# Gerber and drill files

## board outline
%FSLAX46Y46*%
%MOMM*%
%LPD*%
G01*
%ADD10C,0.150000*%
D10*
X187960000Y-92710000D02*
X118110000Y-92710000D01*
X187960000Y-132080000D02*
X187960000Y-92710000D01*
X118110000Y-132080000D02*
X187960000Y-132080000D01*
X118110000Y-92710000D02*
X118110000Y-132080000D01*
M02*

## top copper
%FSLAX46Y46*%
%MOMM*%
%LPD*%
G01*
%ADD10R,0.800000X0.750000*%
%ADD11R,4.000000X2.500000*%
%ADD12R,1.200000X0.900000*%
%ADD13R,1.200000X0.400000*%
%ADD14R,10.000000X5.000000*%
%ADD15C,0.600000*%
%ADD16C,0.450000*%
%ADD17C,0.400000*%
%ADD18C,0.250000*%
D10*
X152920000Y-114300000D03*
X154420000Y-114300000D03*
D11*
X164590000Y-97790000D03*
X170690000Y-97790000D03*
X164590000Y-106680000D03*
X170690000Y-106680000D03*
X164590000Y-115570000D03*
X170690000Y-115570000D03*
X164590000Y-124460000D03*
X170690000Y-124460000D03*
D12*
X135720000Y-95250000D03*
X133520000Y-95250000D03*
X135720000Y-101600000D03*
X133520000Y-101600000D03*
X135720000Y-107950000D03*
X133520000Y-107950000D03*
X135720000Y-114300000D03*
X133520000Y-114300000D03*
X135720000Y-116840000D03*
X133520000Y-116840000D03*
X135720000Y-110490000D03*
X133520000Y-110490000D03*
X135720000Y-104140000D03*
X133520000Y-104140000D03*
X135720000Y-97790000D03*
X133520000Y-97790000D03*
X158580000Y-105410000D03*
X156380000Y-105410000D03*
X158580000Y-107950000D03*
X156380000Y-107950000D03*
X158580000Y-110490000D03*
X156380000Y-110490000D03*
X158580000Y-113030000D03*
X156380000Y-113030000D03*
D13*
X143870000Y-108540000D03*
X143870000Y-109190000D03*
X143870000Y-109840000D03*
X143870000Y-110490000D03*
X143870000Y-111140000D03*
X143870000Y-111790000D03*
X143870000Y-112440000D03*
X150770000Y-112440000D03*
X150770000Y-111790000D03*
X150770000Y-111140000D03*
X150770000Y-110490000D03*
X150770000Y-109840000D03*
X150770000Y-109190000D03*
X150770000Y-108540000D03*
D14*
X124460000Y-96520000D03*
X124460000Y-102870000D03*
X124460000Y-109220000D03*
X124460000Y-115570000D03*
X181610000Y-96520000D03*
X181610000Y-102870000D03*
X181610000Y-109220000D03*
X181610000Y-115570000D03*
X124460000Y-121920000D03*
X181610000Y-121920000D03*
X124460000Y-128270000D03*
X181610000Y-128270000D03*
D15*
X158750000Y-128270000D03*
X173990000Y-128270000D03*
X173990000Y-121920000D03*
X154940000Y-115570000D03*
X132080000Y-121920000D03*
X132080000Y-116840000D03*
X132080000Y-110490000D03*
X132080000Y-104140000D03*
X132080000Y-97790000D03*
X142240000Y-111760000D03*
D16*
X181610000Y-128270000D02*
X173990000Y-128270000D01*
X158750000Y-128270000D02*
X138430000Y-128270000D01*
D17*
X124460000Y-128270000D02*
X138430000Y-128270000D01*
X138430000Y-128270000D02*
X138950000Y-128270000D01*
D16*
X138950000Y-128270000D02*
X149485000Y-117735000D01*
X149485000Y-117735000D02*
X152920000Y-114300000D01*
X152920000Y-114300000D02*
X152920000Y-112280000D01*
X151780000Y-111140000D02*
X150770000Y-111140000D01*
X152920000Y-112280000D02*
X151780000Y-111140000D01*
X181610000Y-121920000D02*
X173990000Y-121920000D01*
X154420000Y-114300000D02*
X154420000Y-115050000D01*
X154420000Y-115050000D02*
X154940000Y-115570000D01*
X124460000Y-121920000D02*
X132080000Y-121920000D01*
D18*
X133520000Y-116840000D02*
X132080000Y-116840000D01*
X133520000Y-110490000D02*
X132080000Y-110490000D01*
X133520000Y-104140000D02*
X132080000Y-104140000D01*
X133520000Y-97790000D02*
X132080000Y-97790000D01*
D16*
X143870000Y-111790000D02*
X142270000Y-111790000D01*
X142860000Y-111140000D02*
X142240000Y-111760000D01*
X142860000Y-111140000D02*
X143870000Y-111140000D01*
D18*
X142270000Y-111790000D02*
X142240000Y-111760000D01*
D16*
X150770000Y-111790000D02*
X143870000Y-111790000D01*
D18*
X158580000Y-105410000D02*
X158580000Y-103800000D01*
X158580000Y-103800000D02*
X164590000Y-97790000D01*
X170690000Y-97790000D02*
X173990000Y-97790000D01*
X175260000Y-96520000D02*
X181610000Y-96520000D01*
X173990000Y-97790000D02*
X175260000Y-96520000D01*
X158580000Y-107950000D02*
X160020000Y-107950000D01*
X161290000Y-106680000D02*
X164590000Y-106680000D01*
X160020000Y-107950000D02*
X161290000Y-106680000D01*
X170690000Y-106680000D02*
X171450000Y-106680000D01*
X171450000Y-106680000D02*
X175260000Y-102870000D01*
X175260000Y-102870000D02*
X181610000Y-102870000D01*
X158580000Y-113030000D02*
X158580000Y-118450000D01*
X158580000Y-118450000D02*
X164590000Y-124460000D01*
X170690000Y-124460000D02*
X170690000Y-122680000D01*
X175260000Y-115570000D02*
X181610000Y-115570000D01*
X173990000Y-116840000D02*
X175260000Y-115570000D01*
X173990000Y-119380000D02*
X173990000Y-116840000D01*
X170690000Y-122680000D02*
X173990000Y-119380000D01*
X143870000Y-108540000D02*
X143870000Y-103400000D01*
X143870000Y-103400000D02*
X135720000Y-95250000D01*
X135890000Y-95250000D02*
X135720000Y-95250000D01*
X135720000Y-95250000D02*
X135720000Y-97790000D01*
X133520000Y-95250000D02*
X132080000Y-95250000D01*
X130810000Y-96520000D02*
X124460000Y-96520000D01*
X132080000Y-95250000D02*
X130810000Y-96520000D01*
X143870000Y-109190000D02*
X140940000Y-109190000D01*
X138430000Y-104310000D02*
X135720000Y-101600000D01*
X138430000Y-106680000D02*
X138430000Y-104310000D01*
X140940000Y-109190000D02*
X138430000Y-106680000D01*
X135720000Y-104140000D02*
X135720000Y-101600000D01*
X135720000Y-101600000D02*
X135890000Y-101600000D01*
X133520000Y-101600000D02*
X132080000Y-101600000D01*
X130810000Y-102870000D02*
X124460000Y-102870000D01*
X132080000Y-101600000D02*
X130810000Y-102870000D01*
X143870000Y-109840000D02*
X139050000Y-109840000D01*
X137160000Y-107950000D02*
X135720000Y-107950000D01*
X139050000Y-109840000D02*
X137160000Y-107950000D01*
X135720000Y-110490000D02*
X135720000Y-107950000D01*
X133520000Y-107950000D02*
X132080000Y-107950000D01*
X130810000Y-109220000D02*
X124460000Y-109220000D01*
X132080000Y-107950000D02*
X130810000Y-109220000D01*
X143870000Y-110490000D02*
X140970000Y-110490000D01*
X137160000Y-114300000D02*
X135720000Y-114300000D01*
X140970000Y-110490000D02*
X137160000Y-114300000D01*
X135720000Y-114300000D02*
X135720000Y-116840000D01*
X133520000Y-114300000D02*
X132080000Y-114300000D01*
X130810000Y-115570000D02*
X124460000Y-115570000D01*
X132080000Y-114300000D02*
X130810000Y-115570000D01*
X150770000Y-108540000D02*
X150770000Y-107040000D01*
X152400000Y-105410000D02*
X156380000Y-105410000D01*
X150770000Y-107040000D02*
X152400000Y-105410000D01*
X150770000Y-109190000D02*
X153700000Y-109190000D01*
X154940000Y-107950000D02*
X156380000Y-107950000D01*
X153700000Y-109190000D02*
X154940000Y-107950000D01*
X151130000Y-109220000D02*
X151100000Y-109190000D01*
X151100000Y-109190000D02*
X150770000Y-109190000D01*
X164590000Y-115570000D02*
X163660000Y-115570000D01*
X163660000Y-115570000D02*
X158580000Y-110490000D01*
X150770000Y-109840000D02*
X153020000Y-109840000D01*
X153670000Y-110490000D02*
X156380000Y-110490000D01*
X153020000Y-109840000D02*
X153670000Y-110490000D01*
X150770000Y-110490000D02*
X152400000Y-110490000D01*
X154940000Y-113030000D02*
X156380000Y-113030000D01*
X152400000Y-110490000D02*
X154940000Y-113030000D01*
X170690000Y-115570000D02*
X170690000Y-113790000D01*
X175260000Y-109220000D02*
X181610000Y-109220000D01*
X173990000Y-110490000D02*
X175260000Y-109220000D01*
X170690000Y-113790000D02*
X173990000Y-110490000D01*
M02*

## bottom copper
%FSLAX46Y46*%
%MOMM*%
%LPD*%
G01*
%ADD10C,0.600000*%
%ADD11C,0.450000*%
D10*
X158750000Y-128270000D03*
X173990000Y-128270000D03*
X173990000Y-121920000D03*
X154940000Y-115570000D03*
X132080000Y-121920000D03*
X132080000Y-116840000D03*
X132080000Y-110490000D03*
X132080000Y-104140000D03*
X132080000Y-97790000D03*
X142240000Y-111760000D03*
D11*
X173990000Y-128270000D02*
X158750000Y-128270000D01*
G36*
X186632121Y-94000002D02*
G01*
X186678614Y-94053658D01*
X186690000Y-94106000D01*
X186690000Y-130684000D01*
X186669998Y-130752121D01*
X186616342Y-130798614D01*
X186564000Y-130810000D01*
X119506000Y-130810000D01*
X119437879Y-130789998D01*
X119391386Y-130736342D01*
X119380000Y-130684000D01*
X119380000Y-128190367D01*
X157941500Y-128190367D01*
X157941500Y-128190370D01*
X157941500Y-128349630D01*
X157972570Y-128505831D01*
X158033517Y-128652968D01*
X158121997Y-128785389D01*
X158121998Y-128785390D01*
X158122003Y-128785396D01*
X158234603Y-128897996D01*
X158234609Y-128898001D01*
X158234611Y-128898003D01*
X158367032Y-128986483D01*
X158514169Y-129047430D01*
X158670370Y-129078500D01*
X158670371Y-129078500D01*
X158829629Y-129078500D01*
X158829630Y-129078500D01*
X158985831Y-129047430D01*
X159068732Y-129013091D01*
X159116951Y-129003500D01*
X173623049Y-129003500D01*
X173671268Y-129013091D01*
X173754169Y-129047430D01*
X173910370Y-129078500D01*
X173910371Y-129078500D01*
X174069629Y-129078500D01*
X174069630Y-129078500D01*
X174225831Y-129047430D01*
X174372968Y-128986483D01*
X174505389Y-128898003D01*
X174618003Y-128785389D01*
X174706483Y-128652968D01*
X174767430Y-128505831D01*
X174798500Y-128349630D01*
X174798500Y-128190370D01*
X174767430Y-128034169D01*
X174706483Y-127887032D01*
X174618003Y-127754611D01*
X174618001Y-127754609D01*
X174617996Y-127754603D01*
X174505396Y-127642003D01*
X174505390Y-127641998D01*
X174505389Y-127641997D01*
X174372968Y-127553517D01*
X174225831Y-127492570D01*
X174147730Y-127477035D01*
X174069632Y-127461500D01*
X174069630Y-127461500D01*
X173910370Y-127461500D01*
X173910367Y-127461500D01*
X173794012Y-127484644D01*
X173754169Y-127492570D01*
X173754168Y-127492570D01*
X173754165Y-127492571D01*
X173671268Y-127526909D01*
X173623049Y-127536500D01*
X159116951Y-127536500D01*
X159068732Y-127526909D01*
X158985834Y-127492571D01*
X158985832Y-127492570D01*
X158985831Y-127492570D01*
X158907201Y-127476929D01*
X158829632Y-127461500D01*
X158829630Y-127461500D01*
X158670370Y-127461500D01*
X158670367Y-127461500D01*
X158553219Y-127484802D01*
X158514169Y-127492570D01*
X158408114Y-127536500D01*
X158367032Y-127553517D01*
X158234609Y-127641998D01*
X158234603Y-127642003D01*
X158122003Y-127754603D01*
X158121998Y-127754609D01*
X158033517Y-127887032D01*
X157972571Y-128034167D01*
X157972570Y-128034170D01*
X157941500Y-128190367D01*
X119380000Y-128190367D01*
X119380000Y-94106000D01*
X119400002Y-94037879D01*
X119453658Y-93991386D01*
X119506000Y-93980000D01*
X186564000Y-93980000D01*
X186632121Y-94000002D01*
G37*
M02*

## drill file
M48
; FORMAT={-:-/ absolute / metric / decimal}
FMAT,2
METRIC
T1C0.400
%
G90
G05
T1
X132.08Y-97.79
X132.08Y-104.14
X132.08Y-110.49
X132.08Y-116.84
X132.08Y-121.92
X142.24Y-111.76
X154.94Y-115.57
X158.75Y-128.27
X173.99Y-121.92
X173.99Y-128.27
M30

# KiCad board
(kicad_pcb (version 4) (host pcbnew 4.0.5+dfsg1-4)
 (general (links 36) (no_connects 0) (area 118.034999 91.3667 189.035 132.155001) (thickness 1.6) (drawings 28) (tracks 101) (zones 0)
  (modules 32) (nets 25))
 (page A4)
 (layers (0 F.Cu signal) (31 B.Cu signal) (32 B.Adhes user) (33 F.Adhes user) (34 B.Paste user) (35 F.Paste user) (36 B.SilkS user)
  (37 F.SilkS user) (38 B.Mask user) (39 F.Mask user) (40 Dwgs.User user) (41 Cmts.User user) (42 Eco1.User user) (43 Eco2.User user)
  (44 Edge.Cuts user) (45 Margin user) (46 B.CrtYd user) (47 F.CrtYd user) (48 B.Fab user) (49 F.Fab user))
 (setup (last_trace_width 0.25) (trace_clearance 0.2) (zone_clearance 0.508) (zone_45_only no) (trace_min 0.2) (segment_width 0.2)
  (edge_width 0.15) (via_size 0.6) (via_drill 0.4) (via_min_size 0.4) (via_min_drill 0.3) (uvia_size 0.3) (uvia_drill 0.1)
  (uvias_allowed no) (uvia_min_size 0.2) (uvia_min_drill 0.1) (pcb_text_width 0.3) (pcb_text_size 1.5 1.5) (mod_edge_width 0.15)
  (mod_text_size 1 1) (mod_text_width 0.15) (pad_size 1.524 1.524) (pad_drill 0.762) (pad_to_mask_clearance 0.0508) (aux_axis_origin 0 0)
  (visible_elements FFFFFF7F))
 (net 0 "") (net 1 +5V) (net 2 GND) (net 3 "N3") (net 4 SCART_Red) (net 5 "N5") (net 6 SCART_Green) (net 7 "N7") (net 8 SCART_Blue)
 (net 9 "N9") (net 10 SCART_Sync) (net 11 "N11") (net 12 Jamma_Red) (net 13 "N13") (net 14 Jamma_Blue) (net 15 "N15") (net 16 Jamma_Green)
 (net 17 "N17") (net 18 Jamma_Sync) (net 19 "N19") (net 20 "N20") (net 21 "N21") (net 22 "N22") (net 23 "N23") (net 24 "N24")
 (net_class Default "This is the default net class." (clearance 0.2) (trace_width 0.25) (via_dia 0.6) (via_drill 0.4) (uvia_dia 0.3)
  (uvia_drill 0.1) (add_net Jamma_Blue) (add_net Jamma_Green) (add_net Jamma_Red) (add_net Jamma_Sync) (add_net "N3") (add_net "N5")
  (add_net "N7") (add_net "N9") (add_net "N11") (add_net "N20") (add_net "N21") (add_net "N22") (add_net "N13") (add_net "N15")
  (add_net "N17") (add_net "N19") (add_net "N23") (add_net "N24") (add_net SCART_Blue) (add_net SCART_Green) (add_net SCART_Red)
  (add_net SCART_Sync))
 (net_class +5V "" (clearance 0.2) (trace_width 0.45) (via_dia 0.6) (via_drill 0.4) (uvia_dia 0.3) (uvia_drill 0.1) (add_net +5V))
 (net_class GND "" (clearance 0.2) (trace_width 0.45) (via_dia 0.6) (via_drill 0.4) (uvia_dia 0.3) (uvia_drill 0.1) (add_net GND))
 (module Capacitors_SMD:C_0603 (layer F.Cu) (at 153.67 114.3)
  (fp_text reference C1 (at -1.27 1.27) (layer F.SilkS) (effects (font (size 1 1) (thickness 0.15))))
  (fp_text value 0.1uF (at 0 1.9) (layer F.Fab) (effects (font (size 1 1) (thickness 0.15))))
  (pad 1 smd rect (at -0.75 0) (size 0.8 0.75) (layers F.Cu F.Paste F.Mask) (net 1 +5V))
  (pad 2 smd rect (at 0.75 0) (size 0.8 0.75) (layers F.Cu F.Paste F.Mask) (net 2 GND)))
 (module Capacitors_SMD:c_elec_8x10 (layer F.Cu) (at 167.64 97.79)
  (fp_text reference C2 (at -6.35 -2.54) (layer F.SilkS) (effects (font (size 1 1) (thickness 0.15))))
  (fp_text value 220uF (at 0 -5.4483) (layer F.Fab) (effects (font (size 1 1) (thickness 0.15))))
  (pad 1 smd rect (at -3.05 0 180) (size 4 2.5) (layers F.Cu F.Paste F.Mask) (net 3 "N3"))
  (pad 2 smd rect (at 3.05 0 180) (size 4 2.5) (layers F.Cu F.Paste F.Mask) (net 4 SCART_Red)))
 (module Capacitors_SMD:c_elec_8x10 (layer F.Cu) (at 167.64 106.68)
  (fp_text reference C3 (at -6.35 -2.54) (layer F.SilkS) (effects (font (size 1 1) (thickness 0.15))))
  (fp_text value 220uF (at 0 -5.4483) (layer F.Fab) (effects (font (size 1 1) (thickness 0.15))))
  (pad 1 smd rect (at -3.05 0 180) (size 4 2.5) (layers F.Cu F.Paste F.Mask) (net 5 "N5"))
  (pad 2 smd rect (at 3.05 0 180) (size 4 2.5) (layers F.Cu F.Paste F.Mask) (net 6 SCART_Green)))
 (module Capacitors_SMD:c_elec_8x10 (layer F.Cu) (at 167.64 115.57)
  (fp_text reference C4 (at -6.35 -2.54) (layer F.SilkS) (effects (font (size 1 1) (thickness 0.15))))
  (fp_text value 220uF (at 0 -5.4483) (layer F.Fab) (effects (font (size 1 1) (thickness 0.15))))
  (pad 1 smd rect (at -3.05 0 180) (size 4 2.5) (layers F.Cu F.Paste F.Mask) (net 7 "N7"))
  (pad 2 smd rect (at 3.05 0 180) (size 4 2.5) (layers F.Cu F.Paste F.Mask) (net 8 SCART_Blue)))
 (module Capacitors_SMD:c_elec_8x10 (layer F.Cu) (at 167.64 124.46)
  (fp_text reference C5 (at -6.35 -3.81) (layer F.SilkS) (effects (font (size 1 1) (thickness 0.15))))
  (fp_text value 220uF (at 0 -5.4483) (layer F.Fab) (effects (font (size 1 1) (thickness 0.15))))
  (pad 1 smd rect (at -3.05 0 180) (size 4 2.5) (layers F.Cu F.Paste F.Mask) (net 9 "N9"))
  (pad 2 smd rect (at 3.05 0 180) (size 4 2.5) (layers F.Cu F.Paste F.Mask) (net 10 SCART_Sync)))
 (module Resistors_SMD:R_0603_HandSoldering (layer F.Cu) (at 134.62 95.25 180)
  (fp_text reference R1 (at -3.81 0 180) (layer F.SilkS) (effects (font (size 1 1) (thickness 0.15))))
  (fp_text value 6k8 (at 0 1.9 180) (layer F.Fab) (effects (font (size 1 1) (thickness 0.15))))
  (pad 1 smd rect (at -1.1 0 180) (size 1.2 0.9) (layers F.Cu F.Paste F.Mask) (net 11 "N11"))
  (pad 2 smd rect (at 1.1 0 180) (size 1.2 0.9) (layers F.Cu F.Paste F.Mask) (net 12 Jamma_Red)))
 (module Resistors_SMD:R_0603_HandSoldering (layer F.Cu) (at 134.62 101.6 180)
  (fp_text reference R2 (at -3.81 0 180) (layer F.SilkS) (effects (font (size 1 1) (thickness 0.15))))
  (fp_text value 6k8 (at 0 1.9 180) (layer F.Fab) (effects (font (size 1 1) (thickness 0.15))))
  (pad 1 smd rect (at -1.1 0 180) (size 1.2 0.9) (layers F.Cu F.Paste F.Mask) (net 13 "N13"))
  (pad 2 smd rect (at 1.1 0 180) (size 1.2 0.9) (layers F.Cu F.Paste F.Mask) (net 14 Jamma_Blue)))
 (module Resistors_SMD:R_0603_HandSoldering (layer F.Cu) (at 134.62 107.95 180)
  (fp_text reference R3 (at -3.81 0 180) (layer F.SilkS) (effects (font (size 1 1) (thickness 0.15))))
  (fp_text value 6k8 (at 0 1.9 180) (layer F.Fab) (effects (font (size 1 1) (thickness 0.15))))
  (pad 1 smd rect (at -1.1 0 180) (size 1.2 0.9) (layers F.Cu F.Paste F.Mask) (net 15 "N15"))
  (pad 2 smd rect (at 1.1 0 180) (size 1.2 0.9) (layers F.Cu F.Paste F.Mask) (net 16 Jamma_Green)))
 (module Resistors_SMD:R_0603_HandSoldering (layer F.Cu) (at 134.62 114.3 180)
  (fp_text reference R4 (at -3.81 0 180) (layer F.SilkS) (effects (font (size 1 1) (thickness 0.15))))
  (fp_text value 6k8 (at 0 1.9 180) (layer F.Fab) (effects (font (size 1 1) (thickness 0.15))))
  (pad 1 smd rect (at -1.1 0 180) (size 1.2 0.9) (layers F.Cu F.Paste F.Mask) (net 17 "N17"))
  (pad 2 smd rect (at 1.1 0 180) (size 1.2 0.9) (layers F.Cu F.Paste F.Mask) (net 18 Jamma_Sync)))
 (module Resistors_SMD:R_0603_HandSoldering (layer F.Cu) (at 134.62 116.84 180)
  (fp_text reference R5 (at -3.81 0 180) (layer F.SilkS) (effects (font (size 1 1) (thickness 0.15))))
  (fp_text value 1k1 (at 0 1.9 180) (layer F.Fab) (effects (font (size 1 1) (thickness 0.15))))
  (pad 1 smd rect (at -1.1 0 180) (size 1.2 0.9) (layers F.Cu F.Paste F.Mask) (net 17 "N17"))
  (pad 2 smd rect (at 1.1 0 180) (size 1.2 0.9) (layers F.Cu F.Paste F.Mask) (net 2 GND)))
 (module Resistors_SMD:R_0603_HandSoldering (layer F.Cu) (at 134.62 110.49 180)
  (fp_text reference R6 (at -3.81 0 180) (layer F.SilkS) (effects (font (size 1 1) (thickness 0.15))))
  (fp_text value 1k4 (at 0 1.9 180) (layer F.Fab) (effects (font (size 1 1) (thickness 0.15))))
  (pad 1 smd rect (at -1.1 0 180) (size 1.2 0.9) (layers F.Cu F.Paste F.Mask) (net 15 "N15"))
  (pad 2 smd rect (at 1.1 0 180) (size 1.2 0.9) (layers F.Cu F.Paste F.Mask) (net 2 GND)))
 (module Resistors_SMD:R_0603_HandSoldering (layer F.Cu) (at 134.62 104.14 180)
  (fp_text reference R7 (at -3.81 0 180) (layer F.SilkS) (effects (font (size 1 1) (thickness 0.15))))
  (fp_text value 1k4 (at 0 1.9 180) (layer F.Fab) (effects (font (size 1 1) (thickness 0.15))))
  (pad 1 smd rect (at -1.1 0 180) (size 1.2 0.9) (layers F.Cu F.Paste F.Mask) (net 13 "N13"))
  (pad 2 smd rect (at 1.1 0 180) (size 1.2 0.9) (layers F.Cu F.Paste F.Mask) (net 2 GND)))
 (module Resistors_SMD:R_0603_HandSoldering (layer F.Cu) (at 134.62 97.79 180)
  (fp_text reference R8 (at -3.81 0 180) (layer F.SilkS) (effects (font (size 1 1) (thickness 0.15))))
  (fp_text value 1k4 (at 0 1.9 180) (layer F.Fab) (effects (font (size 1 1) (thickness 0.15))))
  (pad 1 smd rect (at -1.1 0 180) (size 1.2 0.9) (layers F.Cu F.Paste F.Mask) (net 11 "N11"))
  (pad 2 smd rect (at 1.1 0 180) (size 1.2 0.9) (layers F.Cu F.Paste F.Mask) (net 2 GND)))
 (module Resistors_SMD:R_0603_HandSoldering (layer F.Cu) (at 157.48 105.41 180)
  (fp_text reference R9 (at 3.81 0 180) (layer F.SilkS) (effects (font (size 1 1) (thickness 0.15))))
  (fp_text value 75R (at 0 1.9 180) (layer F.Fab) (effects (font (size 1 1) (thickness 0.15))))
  (pad 1 smd rect (at -1.1 0 180) (size 1.2 0.9) (layers F.Cu F.Paste F.Mask) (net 3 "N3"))
  (pad 2 smd rect (at 1.1 0 180) (size 1.2 0.9) (layers F.Cu F.Paste F.Mask) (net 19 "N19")))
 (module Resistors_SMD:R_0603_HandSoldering (layer F.Cu) (at 157.48 107.95 180)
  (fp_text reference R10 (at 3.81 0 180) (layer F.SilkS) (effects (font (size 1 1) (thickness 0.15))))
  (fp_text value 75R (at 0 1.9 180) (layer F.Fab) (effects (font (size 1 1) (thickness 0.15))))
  (pad 1 smd rect (at -1.1 0 180) (size 1.2 0.9) (layers F.Cu F.Paste F.Mask) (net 5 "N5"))
  (pad 2 smd rect (at 1.1 0 180) (size 1.2 0.9) (layers F.Cu F.Paste F.Mask) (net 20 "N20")))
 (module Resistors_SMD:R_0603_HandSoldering (layer F.Cu) (at 157.48 110.49 180)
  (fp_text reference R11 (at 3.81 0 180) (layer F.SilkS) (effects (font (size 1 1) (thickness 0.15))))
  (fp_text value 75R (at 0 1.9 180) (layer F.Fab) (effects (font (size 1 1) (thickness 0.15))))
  (pad 1 smd rect (at -1.1 0 180) (size 1.2 0.9) (layers F.Cu F.Paste F.Mask) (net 7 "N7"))
  (pad 2 smd rect (at 1.1 0 180) (size 1.2 0.9) (layers F.Cu F.Paste F.Mask) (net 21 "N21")))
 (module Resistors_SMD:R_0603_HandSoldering (layer F.Cu) (at 157.48 113.03 180)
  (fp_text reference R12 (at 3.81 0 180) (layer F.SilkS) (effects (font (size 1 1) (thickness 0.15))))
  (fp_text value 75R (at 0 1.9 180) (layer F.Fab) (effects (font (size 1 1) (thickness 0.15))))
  (pad 1 smd rect (at -1.1 0 180) (size 1.2 0.9) (layers F.Cu F.Paste F.Mask) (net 9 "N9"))
  (pad 2 smd rect (at 1.1 0 180) (size 1.2 0.9) (layers F.Cu F.Paste F.Mask) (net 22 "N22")))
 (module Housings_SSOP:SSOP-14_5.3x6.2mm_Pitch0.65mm (layer F.Cu) (at 147.32 110.49)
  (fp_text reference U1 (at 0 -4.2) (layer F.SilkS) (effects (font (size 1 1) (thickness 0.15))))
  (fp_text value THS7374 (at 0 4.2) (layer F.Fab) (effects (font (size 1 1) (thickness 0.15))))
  (pad 1 smd rect (at -3.45 -1.95) (size 1.2 0.4) (layers F.Cu F.Paste F.Mask) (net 11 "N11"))
  (pad 2 smd rect (at -3.45 -1.3) (size 1.2 0.4) (layers F.Cu F.Paste F.Mask) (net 13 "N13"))
  (pad 3 smd rect (at -3.45 -0.65) (size 1.2 0.4) (layers F.Cu F.Paste F.Mask) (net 15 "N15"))
  (pad 4 smd rect (at -3.45 0) (size 1.2 0.4) (layers F.Cu F.Paste F.Mask) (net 17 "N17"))
  (pad 5 smd rect (at -3.45 0.65) (size 1.2 0.4) (layers F.Cu F.Paste F.Mask) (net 2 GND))
  (pad 6 smd rect (at -3.45 1.3) (size 1.2 0.4) (layers F.Cu F.Paste F.Mask) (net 2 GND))
  (pad 7 smd rect (at -3.45 1.95) (size 1.2 0.4) (layers F.Cu F.Paste F.Mask) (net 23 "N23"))
  (pad 8 smd rect (at 3.45 1.95) (size 1.2 0.4) (layers F.Cu F.Paste F.Mask) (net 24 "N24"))
  (pad 9 smd rect (at 3.45 1.3) (size 1.2 0.4) (layers F.Cu F.Paste F.Mask) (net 2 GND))
  (pad 10 smd rect (at 3.45 0.65) (size 1.2 0.4) (layers F.Cu F.Paste F.Mask) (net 1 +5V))
  (pad 11 smd rect (at 3.45 0) (size 1.2 0.4) (layers F.Cu F.Paste F.Mask) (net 22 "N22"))
  (pad 12 smd rect (at 3.45 -0.65) (size 1.2 0.4) (layers F.Cu F.Paste F.Mask) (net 21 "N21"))
  (pad 13 smd rect (at 3.45 -1.3) (size 1.2 0.4) (layers F.Cu F.Paste F.Mask) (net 20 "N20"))
  (pad 14 smd rect (at 3.45 -1.95) (size 1.2 0.4) (layers F.Cu F.Paste F.Mask) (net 19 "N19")))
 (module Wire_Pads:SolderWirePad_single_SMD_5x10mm (layer F.Cu) (at 124.46 96.52 90)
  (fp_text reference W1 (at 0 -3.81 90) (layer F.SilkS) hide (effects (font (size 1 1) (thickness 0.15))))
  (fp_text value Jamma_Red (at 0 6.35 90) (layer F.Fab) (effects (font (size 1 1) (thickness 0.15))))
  (pad 1 smd rect (at 0 0 90) (size 5 10) (layers F.Cu F.Paste F.Mask) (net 12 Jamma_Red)))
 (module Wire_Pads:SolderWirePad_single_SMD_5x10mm (layer F.Cu) (at 124.46 102.87 90)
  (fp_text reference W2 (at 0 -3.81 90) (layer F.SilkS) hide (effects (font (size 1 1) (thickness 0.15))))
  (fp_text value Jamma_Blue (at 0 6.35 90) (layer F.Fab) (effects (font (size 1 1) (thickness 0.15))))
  (pad 1 smd rect (at 0 0 90) (size 5 10) (layers F.Cu F.Paste F.Mask) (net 14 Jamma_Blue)))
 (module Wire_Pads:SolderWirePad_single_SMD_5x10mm (layer F.Cu) (at 124.46 109.22 90)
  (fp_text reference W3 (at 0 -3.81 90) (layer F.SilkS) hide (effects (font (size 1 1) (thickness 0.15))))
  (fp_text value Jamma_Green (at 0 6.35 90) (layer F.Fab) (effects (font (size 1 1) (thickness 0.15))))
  (pad 1 smd rect (at 0 0 90) (size 5 10) (layers F.Cu F.Paste F.Mask) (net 16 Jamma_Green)))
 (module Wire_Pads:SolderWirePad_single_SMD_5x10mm (layer F.Cu) (at 124.46 115.57 90)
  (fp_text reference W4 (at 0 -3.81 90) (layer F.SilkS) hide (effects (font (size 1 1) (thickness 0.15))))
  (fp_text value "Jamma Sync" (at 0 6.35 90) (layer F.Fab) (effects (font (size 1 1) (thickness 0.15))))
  (pad 1 smd rect (at 0 0 90) (size 5 10) (layers F.Cu F.Paste F.Mask) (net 18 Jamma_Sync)))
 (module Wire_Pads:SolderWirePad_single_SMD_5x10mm (layer F.Cu) (at 181.61 96.52 90)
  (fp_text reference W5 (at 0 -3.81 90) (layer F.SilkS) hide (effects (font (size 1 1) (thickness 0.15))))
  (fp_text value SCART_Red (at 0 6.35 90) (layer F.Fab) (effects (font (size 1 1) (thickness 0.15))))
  (pad 1 smd rect (at 0 0 90) (size 5 10) (layers F.Cu F.Paste F.Mask) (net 4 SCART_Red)))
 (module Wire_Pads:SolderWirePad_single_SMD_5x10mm (layer F.Cu) (at 181.61 102.87 90)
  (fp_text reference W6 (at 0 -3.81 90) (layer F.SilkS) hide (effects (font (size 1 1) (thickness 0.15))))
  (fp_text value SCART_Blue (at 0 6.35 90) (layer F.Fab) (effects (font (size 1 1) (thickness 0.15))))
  (pad 1 smd rect (at 0 0 90) (size 5 10) (layers F.Cu F.Paste F.Mask) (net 6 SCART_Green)))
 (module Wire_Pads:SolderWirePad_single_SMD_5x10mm (layer F.Cu) (at 181.61 109.22 90)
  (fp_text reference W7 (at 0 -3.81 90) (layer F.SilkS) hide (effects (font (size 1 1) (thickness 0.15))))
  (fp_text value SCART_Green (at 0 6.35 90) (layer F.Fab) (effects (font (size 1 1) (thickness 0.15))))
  (pad 1 smd rect (at 0 0 90) (size 5 10) (layers F.Cu F.Paste F.Mask) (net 8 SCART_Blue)))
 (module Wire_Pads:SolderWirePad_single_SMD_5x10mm (layer F.Cu) (at 181.61 115.57 90)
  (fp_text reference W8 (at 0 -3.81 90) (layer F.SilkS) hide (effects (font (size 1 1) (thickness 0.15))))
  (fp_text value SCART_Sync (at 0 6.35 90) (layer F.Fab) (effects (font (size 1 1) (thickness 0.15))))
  (pad 1 smd rect (at 0 0 90) (size 5 10) (layers F.Cu F.Paste F.Mask) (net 10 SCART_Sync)))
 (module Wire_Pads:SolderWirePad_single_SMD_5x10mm (layer F.Cu) (at 124.46 121.92 90)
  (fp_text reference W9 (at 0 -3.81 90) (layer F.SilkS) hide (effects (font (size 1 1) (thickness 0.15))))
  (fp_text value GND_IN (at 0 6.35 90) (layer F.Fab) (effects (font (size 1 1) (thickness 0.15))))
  (pad 1 smd rect (at 0 0 90) (size 5 10) (layers F.Cu F.Paste F.Mask) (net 2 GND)))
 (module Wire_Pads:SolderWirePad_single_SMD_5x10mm (layer F.Cu) (at 181.61 121.92 90)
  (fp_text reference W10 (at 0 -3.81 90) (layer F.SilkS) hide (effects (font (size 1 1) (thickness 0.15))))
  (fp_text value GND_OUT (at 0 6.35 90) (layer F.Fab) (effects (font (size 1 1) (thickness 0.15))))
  (pad 1 smd rect (at 0 0 90) (size 5 10) (layers F.Cu F.Paste F.Mask) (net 2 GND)))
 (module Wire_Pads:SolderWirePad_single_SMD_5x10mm (layer F.Cu) (at 124.46 128.27 90)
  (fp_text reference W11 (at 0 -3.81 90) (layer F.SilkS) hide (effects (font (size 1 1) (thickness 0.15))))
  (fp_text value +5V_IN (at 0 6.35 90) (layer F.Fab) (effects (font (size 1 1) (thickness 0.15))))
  (pad 1 smd rect (at 0 0 90) (size 5 10) (layers F.Cu F.Paste F.Mask) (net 1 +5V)))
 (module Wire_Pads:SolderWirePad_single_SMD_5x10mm (layer F.Cu) (at 181.61 128.27 90)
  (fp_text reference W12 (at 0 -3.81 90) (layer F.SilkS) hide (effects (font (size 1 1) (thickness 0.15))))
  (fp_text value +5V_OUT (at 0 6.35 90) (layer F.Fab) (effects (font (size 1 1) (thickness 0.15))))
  (pad 1 smd rect (at 0 0 90) (size 5 10) (layers F.Cu F.Paste F.Mask) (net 1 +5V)))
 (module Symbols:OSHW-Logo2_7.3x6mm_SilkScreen (layer F.Cu) (at 158.75 124.46)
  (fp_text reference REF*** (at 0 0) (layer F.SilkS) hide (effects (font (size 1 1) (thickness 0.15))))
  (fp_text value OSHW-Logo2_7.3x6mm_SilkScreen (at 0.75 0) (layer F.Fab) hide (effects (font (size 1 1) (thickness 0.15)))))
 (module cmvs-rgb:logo (layer B.Cu) (at 170.18 119.38 180)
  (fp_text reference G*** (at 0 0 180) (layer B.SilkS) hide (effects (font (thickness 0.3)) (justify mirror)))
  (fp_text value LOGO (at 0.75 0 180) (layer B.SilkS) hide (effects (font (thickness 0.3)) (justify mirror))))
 (gr_line (start 187.96 92.71) (end 118.11 92.71) (angle 90) (layer Edge.Cuts) (width 0.15))
 (gr_line (start 187.96 132.08) (end 187.96 92.71) (angle 90) (layer Edge.Cuts) (width 0.15))
 (gr_line (start 118.11 132.08) (end 187.96 132.08) (angle 90) (layer Edge.Cuts) (width 0.15))
 (gr_line (start 118.11 92.71) (end 118.11 132.08) (angle 90) (layer Edge.Cuts) (width 0.15))
 (segment (start 181.61 128.27) (end 173.99 128.27) (width 0.45) (layer F.Cu) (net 1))
 (segment (start 158.75 128.27) (end 138.43 128.27) (width 0.45) (layer F.Cu) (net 1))
 (via (at 158.75 128.27) (size 0.6) (drill 0.4) (layers F.Cu B.Cu) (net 1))
 (segment (start 173.99 128.27) (end 158.75 128.27) (width 0.45) (layer B.Cu) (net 1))
 (via (at 173.99 128.27) (size 0.6) (drill 0.4) (layers F.Cu B.Cu) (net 1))
 (segment (start 124.46 128.27) (end 138.43 128.27) (width 0.4) (layer F.Cu) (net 1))
 (segment (start 138.43 128.27) (end 138.95 128.27) (width 0.4) (layer F.Cu) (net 1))
 (segment (start 138.95 128.27) (end 149.485 117.735) (width 0.45) (layer F.Cu) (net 1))
 (segment (start 149.485 117.735) (end 152.92 114.3) (width 0.45) (layer F.Cu) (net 1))
 (segment (start 152.92 114.3) (end 152.92 112.28) (width 0.45) (layer F.Cu) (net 1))
 (segment (start 151.78 111.14) (end 150.77 111.14) (width 0.45) (layer F.Cu) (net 1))
 (segment (start 152.92 112.28) (end 151.78 111.14) (width 0.45) (layer F.Cu) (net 1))
 (segment (start 181.61 121.92) (end 173.99 121.92) (width 0.45) (layer F.Cu) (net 2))
 (via (at 173.99 121.92) (size 0.6) (drill 0.4) (layers F.Cu B.Cu) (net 2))
 (segment (start 154.42 114.3) (end 154.42 115.05) (width 0.45) (layer F.Cu) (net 2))
 (via (at 154.94 115.57) (size 0.6) (drill 0.4) (layers F.Cu B.Cu) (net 2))
 (segment (start 154.42 115.05) (end 154.94 115.57) (width 0.45) (layer F.Cu) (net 2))
 (segment (start 124.46 121.92) (end 132.08 121.92) (width 0.45) (layer F.Cu) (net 2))
 (via (at 132.08 121.92) (size 0.6) (drill 0.4) (layers F.Cu B.Cu) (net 2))
 (segment (start 133.52 116.84) (end 132.08 116.84) (width 0.25) (layer F.Cu) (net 2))
 (via (at 132.08 116.84) (size 0.6) (drill 0.4) (layers F.Cu B.Cu) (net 2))
 (segment (start 133.52 110.49) (end 132.08 110.49) (width 0.25) (layer F.Cu) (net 2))
 (via (at 132.08 110.49) (size 0.6) (drill 0.4) (layers F.Cu B.Cu) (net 2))
 (segment (start 133.52 104.14) (end 132.08 104.14) (width 0.25) (layer F.Cu) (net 2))
 (via (at 132.08 104.14) (size 0.6) (drill 0.4) (layers F.Cu B.Cu) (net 2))
 (segment (start 133.52 97.79) (end 132.08 97.79) (width 0.25) (layer F.Cu) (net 2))
 (via (at 132.08 97.79) (size 0.6) (drill 0.4) (layers F.Cu B.Cu) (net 2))
 (segment (start 143.87 111.79) (end 142.27 111.79) (width 0.45) (layer F.Cu) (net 2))
 (segment (start 142.86 111.14) (end 142.24 111.76) (width 0.45) (layer F.Cu) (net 2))
 (via (at 142.24 111.76) (size 0.6) (drill 0.4) (layers F.Cu B.Cu) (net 2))
 (segment (start 142.86 111.14) (end 143.87 111.14) (width 0.45) (layer F.Cu) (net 2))
 (segment (start 142.27 111.79) (end 142.24 111.76) (width 0.25) (layer F.Cu) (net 2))
 (segment (start 150.77 111.79) (end 143.87 111.79) (width 0.45) (layer F.Cu) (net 2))
 (segment (start 158.58 105.41) (end 158.58 103.8) (width 0.25) (layer F.Cu) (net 3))
 (segment (start 158.58 103.8) (end 164.59 97.79) (width 0.25) (layer F.Cu) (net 3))
 (segment (start 170.69 97.79) (end 173.99 97.79) (width 0.25) (layer F.Cu) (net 4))
 (segment (start 175.26 96.52) (end 181.61 96.52) (width 0.25) (layer F.Cu) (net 4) (status 20))
 (segment (start 173.99 97.79) (end 175.26 96.52) (width 0.25) (layer F.Cu) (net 4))
 (segment (start 158.58 107.95) (end 160.02 107.95) (width 0.25) (layer F.Cu) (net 5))
 (segment (start 161.29 106.68) (end 164.59 106.68) (width 0.25) (layer F.Cu) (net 5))
 (segment (start 160.02 107.95) (end 161.29 106.68) (width 0.25) (layer F.Cu) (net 5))
 (segment (start 170.69 106.68) (end 171.45 106.68) (width 0.25) (layer F.Cu) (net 6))
 (segment (start 171.45 106.68) (end 175.26 102.87) (width 0.25) (layer F.Cu) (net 6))
 (segment (start 175.26 102.87) (end 181.61 102.87) (width 0.25) (layer F.Cu) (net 6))
 (segment (start 158.58 113.03) (end 158.58 118.45) (width 0.25) (layer F.Cu) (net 9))
 (segment (start 158.58 118.45) (end 164.59 124.46) (width 0.25) (layer F.Cu) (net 9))
 (segment (start 170.69 124.46) (end 170.69 122.68) (width 0.25) (layer F.Cu) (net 10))
 (segment (start 175.26 115.57) (end 181.61 115.57) (width 0.25) (layer F.Cu) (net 10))
 (segment (start 173.99 116.84) (end 175.26 115.57) (width 0.25) (layer F.Cu) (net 10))
 (segment (start 173.99 119.38) (end 173.99 116.84) (width 0.25) (layer F.Cu) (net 10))
 (segment (start 170.69 122.68) (end 173.99 119.38) (width 0.25) (layer F.Cu) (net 10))
 (segment (start 143.87 108.54) (end 143.87 103.4) (width 0.25) (layer F.Cu) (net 11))
 (segment (start 143.87 103.4) (end 135.72 95.25) (width 0.25) (layer F.Cu) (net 11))
 (segment (start 135.89 95.25) (end 135.72 95.25) (width 0.25) (layer F.Cu) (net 11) (status 30))
 (segment (start 135.72 95.25) (end 135.72 97.79) (width 0.25) (layer F.Cu) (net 11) (status 20))
 (segment (start 133.52 95.25) (end 132.08 95.25) (width 0.25) (layer F.Cu) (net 12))
 (segment (start 130.81 96.52) (end 124.46 96.52) (width 0.25) (layer F.Cu) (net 12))
 (segment (start 132.08 95.25) (end 130.81 96.52) (width 0.25) (layer F.Cu) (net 12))
 (segment (start 143.87 109.19) (end 140.94 109.19) (width 0.25) (layer F.Cu) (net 13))
 (segment (start 138.43 104.31) (end 135.72 101.6) (width 0.25) (layer F.Cu) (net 13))
 (segment (start 138.43 106.68) (end 138.43 104.31) (width 0.25) (layer F.Cu) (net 13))
 (segment (start 140.94 109.19) (end 138.43 106.68) (width 0.25) (layer F.Cu) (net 13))
 (segment (start 135.72 104.14) (end 135.72 101.6) (width 0.25) (layer F.Cu) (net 13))
 (segment (start 135.72 101.6) (end 135.89 101.6) (width 0.25) (layer F.Cu) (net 13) (status 30))
 (segment (start 133.52 101.6) (end 132.08 101.6) (width 0.25) (layer F.Cu) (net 14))
 (segment (start 130.81 102.87) (end 124.46 102.87) (width 0.25) (layer F.Cu) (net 14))
 (segment (start 132.08 101.6) (end 130.81 102.87) (width 0.25) (layer F.Cu) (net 14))
 (segment (start 143.87 109.84) (end 139.05 109.84) (width 0.25) (layer F.Cu) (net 15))
 (segment (start 137.16 107.95) (end 135.72 107.95) (width 0.25) (layer F.Cu) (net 15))
 (segment (start 139.05 109.84) (end 137.16 107.95) (width 0.25) (layer F.Cu) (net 15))
 (segment (start 135.72 110.49) (end 135.72 107.95) (width 0.25) (layer F.Cu) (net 15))
 (segment (start 133.52 107.95) (end 132.08 107.95) (width 0.25) (layer F.Cu) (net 16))
 (segment (start 130.81 109.22) (end 124.46 109.22) (width 0.25) (layer F.Cu) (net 16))
 (segment (start 132.08 107.95) (end 130.81 109.22) (width 0.25) (layer F.Cu) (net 16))
 (segment (start 143.87 110.49) (end 140.97 110.49) (width 0.25) (layer F.Cu) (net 17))
 (segment (start 137.16 114.3) (end 135.72 114.3) (width 0.25) (layer F.Cu) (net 17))
 (segment (start 140.97 110.49) (end 137.16 114.3) (width 0.25) (layer F.Cu) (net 17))
 (segment (start 135.72 114.3) (end 135.72 116.84) (width 0.25) (layer F.Cu) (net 17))
 (segment (start 133.52 114.3) (end 132.08 114.3) (width 0.25) (layer F.Cu) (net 18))
 (segment (start 130.81 115.57) (end 124.46 115.57) (width 0.25) (layer F.Cu) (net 18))
 (segment (start 132.08 114.3) (end 130.81 115.57) (width 0.25) (layer F.Cu) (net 18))
 (segment (start 150.77 108.54) (end 150.77 107.04) (width 0.25) (layer F.Cu) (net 19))
 (segment (start 152.4 105.41) (end 156.38 105.41) (width 0.25) (layer F.Cu) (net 19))
 (segment (start 150.77 107.04) (end 152.4 105.41) (width 0.25) (layer F.Cu) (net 19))
 (segment (start 150.77 109.19) (end 153.7 109.19) (width 0.25) (layer F.Cu) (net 20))
 (segment (start 154.94 107.95) (end 156.38 107.95) (width 0.25) (layer F.Cu) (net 20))
 (segment (start 153.7 109.19) (end 154.94 107.95) (width 0.25) (layer F.Cu) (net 20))
 (segment (start 151.13 109.22) (end 151.1 109.19) (width 0.25) (layer F.Cu) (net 20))
 (segment (start 151.1 109.19) (end 150.77 109.19) (width 0.25) (layer F.Cu) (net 20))
 (segment (start 164.59 115.57) (end 163.66 115.57) (width 0.25) (layer F.Cu) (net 7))
 (segment (start 163.66 115.57) (end 158.58 110.49) (width 0.25) (layer F.Cu) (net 7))
 (segment (start 150.77 109.84) (end 153.02 109.84) (width 0.25) (layer F.Cu) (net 21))
 (segment (start 153.67 110.49) (end 156.38 110.49) (width 0.25) (layer F.Cu) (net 21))
 (segment (start 153.02 109.84) (end 153.67 110.49) (width 0.25) (layer F.Cu) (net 21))
 (segment (start 150.77 110.49) (end 152.4 110.49) (width 0.25) (layer F.Cu) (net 22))
 (segment (start 154.94 113.03) (end 156.38 113.03) (width 0.25) (layer F.Cu) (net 22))
 (segment (start 152.4 110.49) (end 154.94 113.03) (width 0.25) (layer F.Cu) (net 22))
 (segment (start 170.69 115.57) (end 170.69 113.79) (width 0.25) (layer F.Cu) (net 8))
 (segment (start 175.26 109.22) (end 181.61 109.22) (width 0.25) (layer F.Cu) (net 8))
 (segment (start 173.99 110.49) (end 175.26 109.22) (width 0.25) (layer F.Cu) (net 8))
 (segment (start 170.69 113.79) (end 173.99 110.49) (width 0.25) (layer F.Cu) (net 8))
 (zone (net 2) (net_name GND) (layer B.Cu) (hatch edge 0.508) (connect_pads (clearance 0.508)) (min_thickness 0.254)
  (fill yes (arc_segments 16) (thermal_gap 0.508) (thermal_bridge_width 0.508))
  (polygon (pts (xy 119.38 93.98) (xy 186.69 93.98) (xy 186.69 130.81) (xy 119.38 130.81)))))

